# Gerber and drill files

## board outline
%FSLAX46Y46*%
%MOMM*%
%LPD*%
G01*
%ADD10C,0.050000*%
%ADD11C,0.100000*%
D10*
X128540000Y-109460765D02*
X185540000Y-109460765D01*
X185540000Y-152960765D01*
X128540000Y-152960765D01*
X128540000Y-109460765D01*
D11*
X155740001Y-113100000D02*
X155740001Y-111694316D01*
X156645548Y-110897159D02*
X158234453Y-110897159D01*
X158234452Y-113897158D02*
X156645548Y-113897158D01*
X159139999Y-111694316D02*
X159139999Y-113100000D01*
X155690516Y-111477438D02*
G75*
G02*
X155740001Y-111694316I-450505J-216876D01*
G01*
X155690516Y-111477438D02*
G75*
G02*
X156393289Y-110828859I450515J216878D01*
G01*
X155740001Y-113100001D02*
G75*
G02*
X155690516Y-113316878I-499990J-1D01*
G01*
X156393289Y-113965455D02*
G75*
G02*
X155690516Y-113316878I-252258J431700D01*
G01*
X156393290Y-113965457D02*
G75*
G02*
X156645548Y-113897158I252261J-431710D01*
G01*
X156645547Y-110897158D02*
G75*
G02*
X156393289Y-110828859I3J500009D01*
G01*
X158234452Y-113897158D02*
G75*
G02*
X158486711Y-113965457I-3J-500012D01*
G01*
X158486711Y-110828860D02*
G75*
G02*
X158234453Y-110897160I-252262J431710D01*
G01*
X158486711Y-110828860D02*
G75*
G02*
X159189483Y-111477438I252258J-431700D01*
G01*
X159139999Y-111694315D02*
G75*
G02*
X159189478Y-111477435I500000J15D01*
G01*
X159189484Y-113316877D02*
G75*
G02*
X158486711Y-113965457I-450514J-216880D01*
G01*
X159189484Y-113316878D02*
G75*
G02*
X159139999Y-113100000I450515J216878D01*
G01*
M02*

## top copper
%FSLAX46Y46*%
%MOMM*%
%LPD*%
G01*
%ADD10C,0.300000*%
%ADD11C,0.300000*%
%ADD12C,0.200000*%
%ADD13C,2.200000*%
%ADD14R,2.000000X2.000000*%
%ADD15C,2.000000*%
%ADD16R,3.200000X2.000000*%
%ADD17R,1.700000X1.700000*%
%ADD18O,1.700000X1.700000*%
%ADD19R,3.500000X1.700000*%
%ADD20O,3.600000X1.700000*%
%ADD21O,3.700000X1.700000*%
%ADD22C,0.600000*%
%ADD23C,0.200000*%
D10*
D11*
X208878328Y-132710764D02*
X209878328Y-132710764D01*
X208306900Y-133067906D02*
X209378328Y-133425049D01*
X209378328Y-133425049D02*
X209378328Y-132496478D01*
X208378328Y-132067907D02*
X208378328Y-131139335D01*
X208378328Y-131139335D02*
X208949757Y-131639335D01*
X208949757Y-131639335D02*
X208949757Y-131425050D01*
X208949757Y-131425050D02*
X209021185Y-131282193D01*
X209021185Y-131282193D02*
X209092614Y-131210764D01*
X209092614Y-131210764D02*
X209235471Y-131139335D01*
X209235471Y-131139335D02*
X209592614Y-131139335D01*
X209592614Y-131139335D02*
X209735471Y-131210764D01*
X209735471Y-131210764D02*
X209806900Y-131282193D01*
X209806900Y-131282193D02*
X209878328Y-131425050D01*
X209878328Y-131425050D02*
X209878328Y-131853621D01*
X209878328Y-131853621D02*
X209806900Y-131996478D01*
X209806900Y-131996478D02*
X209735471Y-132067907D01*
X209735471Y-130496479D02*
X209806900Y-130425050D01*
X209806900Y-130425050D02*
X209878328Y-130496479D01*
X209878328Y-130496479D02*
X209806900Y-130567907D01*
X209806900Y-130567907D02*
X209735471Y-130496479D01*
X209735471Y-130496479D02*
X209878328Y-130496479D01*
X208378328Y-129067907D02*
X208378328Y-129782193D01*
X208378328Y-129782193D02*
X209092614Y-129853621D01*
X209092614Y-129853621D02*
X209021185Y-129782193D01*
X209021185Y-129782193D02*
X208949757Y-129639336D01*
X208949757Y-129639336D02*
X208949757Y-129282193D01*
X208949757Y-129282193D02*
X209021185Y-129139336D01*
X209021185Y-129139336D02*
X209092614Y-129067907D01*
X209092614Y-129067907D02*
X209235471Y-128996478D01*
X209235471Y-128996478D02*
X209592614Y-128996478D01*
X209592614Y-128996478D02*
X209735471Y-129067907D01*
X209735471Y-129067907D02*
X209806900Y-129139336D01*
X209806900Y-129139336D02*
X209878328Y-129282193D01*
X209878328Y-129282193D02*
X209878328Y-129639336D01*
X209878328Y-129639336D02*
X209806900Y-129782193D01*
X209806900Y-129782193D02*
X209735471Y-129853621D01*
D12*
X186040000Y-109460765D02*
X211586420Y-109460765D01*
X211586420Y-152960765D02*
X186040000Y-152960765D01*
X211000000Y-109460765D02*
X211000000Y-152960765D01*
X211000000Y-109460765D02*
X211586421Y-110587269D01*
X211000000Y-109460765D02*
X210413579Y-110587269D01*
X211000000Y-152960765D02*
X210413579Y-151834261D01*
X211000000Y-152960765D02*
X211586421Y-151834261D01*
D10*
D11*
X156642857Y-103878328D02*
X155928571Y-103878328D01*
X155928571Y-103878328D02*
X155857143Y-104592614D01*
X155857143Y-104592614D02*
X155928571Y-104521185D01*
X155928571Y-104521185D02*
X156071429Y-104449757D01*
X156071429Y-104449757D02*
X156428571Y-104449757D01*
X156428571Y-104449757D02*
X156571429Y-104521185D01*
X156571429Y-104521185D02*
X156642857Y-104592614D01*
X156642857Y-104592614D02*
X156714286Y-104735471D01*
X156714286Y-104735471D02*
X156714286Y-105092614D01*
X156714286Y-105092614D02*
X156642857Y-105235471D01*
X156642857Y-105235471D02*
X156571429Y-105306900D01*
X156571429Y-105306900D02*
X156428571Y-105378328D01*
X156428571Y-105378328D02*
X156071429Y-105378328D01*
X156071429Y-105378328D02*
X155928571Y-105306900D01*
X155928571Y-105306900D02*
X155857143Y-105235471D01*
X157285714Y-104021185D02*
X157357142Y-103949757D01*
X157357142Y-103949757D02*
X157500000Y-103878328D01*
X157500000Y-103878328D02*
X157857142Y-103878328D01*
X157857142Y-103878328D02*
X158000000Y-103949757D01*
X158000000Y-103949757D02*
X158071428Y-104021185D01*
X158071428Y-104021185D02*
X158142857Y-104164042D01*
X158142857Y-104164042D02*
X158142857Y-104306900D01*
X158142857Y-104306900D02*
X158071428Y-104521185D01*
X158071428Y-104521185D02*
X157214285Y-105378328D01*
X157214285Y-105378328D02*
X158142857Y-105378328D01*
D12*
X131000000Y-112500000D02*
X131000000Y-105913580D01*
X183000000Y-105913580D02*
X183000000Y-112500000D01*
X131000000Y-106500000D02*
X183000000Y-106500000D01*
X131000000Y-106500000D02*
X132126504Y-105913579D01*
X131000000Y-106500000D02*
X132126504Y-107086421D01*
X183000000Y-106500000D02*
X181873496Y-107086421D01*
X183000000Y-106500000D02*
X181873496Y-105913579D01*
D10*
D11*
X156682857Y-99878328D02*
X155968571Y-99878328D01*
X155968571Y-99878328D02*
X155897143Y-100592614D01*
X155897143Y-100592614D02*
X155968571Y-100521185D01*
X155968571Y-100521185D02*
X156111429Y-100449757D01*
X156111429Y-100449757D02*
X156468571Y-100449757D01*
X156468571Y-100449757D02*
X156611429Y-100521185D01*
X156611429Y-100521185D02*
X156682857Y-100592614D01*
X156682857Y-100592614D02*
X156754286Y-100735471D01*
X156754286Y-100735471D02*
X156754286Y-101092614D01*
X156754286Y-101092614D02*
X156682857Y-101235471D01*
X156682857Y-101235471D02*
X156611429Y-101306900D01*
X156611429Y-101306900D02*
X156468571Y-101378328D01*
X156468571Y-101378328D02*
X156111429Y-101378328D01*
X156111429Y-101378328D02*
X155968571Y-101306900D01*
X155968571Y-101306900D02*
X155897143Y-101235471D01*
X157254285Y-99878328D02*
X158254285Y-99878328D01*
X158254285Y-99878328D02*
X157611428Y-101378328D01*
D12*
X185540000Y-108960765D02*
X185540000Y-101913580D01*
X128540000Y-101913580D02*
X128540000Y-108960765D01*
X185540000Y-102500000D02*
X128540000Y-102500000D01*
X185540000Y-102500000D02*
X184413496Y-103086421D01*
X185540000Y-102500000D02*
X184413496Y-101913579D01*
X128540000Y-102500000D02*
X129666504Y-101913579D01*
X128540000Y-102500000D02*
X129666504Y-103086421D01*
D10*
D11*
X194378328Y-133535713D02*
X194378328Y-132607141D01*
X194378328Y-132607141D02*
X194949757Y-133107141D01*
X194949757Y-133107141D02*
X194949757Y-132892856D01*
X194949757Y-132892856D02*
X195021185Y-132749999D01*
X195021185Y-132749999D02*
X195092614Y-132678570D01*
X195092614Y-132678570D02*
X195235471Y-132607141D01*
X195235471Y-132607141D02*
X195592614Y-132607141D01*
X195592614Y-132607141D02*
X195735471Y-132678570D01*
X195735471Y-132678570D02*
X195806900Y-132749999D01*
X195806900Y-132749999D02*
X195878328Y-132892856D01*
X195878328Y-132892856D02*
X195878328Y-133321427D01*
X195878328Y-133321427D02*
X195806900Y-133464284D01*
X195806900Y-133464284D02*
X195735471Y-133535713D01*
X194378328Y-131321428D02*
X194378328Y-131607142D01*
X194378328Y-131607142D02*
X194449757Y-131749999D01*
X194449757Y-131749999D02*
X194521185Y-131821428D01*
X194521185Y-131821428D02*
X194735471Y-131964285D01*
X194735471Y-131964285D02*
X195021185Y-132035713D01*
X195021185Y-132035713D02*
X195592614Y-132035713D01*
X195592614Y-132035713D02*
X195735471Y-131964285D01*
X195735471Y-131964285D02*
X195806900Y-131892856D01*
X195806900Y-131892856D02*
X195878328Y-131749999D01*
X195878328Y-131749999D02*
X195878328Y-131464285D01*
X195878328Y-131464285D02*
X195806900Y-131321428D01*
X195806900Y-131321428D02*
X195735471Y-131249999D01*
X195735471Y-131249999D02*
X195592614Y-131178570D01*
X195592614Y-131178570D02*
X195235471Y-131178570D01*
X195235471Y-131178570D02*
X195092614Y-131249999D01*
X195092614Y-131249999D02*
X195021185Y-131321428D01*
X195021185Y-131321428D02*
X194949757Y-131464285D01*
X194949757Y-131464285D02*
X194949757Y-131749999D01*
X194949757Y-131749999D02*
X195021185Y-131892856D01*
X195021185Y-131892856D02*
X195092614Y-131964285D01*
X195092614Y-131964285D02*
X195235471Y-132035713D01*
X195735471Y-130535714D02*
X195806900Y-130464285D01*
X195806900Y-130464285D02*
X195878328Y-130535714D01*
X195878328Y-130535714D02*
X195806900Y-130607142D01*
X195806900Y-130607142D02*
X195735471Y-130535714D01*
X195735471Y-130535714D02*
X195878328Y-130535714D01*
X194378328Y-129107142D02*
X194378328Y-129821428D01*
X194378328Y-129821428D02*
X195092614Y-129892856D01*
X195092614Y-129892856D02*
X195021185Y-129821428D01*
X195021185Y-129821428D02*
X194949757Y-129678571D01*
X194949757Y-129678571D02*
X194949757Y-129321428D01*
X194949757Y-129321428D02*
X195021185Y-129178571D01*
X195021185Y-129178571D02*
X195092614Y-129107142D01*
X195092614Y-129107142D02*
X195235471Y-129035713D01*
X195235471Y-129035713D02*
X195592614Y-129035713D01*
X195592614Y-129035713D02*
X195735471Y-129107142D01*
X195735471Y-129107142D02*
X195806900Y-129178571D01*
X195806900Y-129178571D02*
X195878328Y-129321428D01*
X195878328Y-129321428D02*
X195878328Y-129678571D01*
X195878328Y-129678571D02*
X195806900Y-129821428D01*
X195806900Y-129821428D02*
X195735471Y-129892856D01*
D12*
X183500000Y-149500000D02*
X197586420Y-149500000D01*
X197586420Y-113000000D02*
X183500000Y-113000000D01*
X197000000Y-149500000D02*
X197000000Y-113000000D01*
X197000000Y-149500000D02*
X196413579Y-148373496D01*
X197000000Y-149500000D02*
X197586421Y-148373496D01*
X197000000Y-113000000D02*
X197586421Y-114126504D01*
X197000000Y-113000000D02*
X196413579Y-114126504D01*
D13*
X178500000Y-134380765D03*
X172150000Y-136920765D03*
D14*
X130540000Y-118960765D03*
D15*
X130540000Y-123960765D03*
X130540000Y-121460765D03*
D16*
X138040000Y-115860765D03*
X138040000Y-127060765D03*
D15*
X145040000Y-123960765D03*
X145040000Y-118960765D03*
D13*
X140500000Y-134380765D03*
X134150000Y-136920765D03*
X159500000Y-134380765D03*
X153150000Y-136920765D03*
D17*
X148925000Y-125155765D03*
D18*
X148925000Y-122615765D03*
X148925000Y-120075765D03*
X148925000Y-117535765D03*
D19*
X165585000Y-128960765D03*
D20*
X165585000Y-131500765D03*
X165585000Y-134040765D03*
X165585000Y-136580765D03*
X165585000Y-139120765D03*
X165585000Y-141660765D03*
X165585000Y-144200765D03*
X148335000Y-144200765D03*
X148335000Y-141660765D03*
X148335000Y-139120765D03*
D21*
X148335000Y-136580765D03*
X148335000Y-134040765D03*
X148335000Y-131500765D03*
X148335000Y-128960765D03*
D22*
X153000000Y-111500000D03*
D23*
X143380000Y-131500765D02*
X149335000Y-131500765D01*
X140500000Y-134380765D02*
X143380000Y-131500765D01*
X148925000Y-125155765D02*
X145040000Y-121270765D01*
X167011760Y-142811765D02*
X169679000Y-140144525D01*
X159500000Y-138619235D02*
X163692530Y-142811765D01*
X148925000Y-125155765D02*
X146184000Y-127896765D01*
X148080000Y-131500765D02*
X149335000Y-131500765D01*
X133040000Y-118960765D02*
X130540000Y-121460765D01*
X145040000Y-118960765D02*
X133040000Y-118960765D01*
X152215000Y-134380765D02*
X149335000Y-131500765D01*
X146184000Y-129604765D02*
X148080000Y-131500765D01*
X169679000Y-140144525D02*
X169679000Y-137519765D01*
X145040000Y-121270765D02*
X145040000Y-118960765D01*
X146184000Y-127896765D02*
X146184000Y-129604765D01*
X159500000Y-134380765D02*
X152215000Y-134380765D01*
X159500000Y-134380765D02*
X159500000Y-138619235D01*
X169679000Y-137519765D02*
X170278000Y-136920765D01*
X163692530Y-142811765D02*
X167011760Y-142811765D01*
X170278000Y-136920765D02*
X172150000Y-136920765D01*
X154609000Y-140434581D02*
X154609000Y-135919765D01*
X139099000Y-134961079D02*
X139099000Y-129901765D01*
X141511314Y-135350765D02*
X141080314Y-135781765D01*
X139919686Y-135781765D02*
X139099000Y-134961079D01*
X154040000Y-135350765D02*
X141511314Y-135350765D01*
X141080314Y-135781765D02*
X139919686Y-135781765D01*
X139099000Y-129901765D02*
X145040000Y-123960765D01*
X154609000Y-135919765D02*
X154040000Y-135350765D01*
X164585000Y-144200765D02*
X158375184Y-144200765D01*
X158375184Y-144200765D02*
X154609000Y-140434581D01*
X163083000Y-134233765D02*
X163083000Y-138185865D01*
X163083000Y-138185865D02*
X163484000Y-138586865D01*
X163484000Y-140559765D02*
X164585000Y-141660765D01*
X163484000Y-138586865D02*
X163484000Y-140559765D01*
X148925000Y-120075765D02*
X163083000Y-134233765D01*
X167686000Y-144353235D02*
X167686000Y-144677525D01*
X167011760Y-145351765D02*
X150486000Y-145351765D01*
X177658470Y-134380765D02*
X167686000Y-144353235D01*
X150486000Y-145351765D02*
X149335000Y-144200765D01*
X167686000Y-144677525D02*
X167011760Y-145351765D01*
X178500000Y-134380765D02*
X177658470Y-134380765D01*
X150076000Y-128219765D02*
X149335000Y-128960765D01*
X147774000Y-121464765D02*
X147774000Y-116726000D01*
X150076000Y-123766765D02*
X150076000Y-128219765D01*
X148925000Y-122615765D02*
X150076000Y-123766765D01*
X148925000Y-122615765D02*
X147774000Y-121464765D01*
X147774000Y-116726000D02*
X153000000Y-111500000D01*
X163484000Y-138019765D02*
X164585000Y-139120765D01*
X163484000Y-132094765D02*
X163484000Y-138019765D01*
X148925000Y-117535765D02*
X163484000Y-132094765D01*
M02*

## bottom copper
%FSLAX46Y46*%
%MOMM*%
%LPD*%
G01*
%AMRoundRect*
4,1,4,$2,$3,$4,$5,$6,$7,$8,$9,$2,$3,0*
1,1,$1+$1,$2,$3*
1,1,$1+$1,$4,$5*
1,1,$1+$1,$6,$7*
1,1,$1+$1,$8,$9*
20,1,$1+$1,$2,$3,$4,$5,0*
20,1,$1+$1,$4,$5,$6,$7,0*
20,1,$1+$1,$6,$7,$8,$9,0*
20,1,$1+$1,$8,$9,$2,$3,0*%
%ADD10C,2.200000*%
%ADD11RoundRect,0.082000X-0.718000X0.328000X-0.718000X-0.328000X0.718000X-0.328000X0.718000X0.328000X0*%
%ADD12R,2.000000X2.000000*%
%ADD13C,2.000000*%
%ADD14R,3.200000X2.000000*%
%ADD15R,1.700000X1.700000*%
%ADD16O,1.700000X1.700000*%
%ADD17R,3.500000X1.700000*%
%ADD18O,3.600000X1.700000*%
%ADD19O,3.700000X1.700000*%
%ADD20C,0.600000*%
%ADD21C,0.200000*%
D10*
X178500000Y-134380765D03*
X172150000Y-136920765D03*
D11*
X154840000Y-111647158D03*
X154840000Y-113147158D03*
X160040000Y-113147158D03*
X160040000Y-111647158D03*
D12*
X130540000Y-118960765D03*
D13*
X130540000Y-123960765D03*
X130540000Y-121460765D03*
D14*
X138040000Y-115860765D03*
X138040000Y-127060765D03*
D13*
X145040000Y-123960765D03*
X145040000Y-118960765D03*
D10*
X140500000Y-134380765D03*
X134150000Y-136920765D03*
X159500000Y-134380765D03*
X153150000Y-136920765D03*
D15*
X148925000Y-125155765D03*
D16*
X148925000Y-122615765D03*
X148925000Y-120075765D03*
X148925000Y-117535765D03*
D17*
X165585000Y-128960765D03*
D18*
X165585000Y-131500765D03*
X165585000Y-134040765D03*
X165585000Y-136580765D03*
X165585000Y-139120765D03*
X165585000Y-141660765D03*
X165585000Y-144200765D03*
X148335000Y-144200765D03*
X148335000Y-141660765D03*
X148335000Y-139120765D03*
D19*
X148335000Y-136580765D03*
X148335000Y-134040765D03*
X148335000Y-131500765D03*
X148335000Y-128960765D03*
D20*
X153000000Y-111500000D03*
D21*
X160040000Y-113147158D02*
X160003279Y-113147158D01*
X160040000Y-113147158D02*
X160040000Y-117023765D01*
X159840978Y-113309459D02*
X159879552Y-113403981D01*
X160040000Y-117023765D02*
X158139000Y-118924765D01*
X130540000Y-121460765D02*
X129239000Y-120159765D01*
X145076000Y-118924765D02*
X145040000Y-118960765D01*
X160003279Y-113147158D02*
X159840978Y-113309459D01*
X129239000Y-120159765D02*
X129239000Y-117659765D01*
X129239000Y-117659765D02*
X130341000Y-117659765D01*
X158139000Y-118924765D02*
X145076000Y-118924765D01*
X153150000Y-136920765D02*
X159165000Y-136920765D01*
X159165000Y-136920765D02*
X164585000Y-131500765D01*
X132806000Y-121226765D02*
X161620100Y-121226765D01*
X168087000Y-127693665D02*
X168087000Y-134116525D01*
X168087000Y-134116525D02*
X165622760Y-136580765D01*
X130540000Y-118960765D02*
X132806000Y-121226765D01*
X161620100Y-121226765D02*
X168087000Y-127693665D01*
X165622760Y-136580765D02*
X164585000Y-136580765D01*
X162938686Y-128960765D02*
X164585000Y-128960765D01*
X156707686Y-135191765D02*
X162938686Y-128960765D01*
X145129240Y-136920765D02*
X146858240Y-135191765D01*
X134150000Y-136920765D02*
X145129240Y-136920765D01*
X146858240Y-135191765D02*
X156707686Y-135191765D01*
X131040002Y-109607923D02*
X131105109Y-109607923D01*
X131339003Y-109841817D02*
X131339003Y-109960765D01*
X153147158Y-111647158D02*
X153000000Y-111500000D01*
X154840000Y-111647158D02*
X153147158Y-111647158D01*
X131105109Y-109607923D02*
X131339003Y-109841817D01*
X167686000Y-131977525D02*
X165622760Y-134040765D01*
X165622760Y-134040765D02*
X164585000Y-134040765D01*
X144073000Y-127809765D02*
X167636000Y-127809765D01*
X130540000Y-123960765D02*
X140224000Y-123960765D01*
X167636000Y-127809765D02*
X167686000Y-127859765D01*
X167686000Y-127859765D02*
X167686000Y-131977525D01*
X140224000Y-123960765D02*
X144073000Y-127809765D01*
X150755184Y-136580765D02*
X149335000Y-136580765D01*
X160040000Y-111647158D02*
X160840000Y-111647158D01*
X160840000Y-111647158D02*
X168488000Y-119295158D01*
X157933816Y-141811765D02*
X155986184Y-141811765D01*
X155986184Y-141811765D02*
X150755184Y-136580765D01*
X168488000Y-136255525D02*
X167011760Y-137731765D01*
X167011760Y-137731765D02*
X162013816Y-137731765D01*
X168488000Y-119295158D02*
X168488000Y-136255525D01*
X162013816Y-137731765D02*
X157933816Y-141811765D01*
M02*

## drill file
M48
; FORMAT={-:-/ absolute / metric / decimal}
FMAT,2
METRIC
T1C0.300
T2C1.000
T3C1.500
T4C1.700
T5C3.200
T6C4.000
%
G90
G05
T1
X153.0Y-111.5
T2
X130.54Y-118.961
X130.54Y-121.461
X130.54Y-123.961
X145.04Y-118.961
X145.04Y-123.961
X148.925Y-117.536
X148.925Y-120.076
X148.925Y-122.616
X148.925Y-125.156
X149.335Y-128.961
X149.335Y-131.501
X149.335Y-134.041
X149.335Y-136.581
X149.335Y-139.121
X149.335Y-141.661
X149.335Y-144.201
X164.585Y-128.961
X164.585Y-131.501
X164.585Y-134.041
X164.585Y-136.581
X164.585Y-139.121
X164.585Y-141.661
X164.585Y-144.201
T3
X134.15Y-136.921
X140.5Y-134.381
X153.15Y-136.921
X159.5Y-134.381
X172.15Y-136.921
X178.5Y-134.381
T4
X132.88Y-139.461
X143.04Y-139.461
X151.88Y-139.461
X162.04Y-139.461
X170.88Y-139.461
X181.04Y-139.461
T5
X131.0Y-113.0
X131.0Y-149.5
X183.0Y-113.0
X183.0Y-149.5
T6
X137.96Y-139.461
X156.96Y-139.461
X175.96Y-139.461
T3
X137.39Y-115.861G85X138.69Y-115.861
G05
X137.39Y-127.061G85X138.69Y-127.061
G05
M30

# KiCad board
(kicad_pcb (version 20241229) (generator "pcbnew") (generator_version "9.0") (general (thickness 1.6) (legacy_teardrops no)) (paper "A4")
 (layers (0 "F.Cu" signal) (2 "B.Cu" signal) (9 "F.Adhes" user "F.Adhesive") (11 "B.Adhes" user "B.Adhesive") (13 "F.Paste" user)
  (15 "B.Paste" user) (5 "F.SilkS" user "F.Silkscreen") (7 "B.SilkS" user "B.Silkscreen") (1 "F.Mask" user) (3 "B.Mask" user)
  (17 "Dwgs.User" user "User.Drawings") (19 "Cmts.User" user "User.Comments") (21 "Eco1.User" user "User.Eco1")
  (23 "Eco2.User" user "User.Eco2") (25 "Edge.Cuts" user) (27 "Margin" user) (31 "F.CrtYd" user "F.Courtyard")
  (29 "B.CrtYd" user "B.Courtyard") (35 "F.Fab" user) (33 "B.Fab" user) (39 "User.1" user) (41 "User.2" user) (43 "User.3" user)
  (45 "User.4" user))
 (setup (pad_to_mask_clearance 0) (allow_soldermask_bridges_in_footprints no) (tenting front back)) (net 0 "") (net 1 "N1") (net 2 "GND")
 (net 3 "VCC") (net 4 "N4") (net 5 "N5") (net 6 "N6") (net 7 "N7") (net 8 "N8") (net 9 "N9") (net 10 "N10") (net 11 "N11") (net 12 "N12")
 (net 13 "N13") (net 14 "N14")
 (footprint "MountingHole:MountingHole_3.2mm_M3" (layer "F.Cu") (at 183 149.5)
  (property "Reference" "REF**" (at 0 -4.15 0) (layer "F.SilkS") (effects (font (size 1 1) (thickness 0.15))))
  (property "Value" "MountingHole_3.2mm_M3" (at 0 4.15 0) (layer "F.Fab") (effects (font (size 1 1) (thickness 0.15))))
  (pad "" np_thru_hole circle (at 0 0) (size 3.2 3.2) (drill 3.2) (layers "*.Cu" "*.Mask")))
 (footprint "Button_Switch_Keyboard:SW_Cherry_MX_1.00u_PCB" (layer "F.Cu") (at 178.5 134.380765)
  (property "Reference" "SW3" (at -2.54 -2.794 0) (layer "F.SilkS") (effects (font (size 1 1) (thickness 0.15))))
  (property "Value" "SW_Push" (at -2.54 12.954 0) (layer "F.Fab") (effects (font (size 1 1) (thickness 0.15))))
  (pad "" np_thru_hole circle (at -7.62 5.08) (size 1.7 1.7) (drill 1.7) (layers "*.Cu" "*.Mask"))
  (pad "" np_thru_hole circle (at -2.54 5.08) (size 4 4) (drill 4) (layers "*.Cu" "*.Mask"))
  (pad "" np_thru_hole circle (at 2.54 5.08) (size 1.7 1.7) (drill 1.7) (layers "*.Cu" "*.Mask"))
  (pad "1" thru_hole circle (at 0 0) (size 2.2 2.2) (drill 1.5) (layers "*.Cu" "*.Mask") (remove_unused_layers no) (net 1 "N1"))
  (pad "2" thru_hole circle (at -6.35 2.54) (size 2.2 2.2) (drill 1.5) (layers "*.Cu" "*.Mask") (remove_unused_layers no) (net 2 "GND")))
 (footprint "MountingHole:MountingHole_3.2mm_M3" (layer "F.Cu") (at 131 149.5)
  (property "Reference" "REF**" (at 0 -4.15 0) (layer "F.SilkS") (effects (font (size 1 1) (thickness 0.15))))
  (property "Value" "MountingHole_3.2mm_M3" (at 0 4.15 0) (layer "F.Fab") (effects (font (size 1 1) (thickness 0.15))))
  (pad "" np_thru_hole circle (at 0 0) (size 3.2 3.2) (drill 3.2) (layers "*.Cu" "*.Mask")))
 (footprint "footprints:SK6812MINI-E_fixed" (layer "F.Cu") (at 157.439999 112.5)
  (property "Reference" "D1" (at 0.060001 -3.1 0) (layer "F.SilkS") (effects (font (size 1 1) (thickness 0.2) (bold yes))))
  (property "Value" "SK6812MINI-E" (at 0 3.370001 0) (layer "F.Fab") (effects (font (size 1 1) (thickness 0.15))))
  (fp_line (start -1.699998 0.6) (end -1.699998 -0.805684) (stroke (width 0.1) (type solid)) (layer "Edge.Cuts"))
  (fp_line (start -0.794451 -1.602841) (end 0.794454 -1.602841) (stroke (width 0.1) (type solid)) (layer "Edge.Cuts"))
  (fp_line (start 0.794453 1.397158) (end -0.794451 1.397158) (stroke (width 0.1) (type solid)) (layer "Edge.Cuts"))
  (fp_line (start 1.7 -0.805684) (end 1.7 0.6) (stroke (width 0.1) (type solid)) (layer "Edge.Cuts"))
  (fp_arc (start -1.749483 -1.022562) (mid -1.712526 -0.91691) (end -1.699998 -0.805684) (stroke (width 0.1) (type solid))
   (layer "Edge.Cuts"))
  (fp_arc (start -1.749483 -1.022562) (mid -1.63807 -1.606877) (end -1.04671 -1.671141) (stroke (width 0.1) (type solid))
   (layer "Edge.Cuts"))
  (fp_arc (start -1.699998 0.600001) (mid -1.712526 0.711226) (end -1.749483 0.816878) (stroke (width 0.1) (type solid)) (layer "Edge.Cuts"))
  (fp_arc (start -1.04671 1.465455) (mid -1.638069 1.401192) (end -1.749483 0.816878) (stroke (width 0.1) (type solid)) (layer "Edge.Cuts"))
  (fp_arc (start -1.046709 1.465457) (mid -0.925121 1.414535) (end -0.794451 1.397158) (stroke (width 0.1) (type solid)) (layer "Edge.Cuts"))
  (fp_arc (start -0.794452 -1.602842) (mid -0.925122 -1.620219) (end -1.04671 -1.671141) (stroke (width 0.1) (type solid))
   (layer "Edge.Cuts"))
  (fp_arc (start 0.794453 1.397158) (mid 0.925124 1.414535) (end 1.046712 1.465457) (stroke (width 0.1) (type solid)) (layer "Edge.Cuts"))
  (fp_arc (start 1.046712 -1.67114) (mid 0.925124 -1.620218) (end 0.794454 -1.602841) (stroke (width 0.1) (type solid)) (layer "Edge.Cuts"))
  (fp_arc (start 1.046712 -1.67114) (mid 1.638072 -1.606876) (end 1.749485 -1.022562) (stroke (width 0.1) (type solid)) (layer "Edge.Cuts"))
  (fp_arc (start 1.7 -0.805685) (mid 1.712528 -0.91691) (end 1.749485 -1.022562) (stroke (width 0.1) (type solid)) (layer "Edge.Cuts"))
  (fp_arc (start 1.749485 0.816877) (mid 1.638073 1.401193) (end 1.046712 1.465457) (stroke (width 0.1) (type solid)) (layer "Edge.Cuts"))
  (fp_arc (start 1.749485 0.816878) (mid 1.712528 0.711226) (end 1.7 0.6) (stroke (width 0.1) (type solid)) (layer "Edge.Cuts"))
  (pad "1" smd roundrect (at -2.599999 -0.852842 270) (size 0.82 1.6) (layers "B.Cu" "B.Mask" "B.Paste") (roundrect_rratio 0.1)
   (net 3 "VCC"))
  (pad "2" smd roundrect (at -2.599999 0.647158 270) (size 0.82 1.6) (layers "B.Cu" "B.Mask" "B.Paste") (roundrect_rratio 0.1))
  (pad "3" smd roundrect (at 2.600001 0.647158 270) (size 0.82 1.6) (layers "B.Cu" "B.Mask" "B.Paste") (roundrect_rratio 0.1) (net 2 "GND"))
  (pad "4" smd roundrect (at 2.600001 -0.852842 270) (size 0.82 1.6) (layers "B.Cu" "B.Mask" "B.Paste") (roundrect_rratio 0.1) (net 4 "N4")))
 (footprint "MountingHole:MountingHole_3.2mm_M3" (layer "F.Cu") (at 131 113)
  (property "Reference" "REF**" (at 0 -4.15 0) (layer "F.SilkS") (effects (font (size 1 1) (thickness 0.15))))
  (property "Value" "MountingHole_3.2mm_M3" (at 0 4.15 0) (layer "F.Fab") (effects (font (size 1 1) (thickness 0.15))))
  (pad "" np_thru_hole circle (at 0 0) (size 3.2 3.2) (drill 3.2) (layers "*.Cu" "*.Mask")))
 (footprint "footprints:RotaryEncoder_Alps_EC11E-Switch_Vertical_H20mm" (layer "F.Cu") (at 130.54 118.960765)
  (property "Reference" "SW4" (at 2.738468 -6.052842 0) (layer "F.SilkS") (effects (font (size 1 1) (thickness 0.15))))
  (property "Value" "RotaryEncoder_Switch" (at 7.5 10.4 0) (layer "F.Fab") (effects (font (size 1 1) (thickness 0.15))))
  (pad "A" thru_hole rect (at 0 0) (size 2 2) (drill 1) (layers "*.Cu" "*.Mask") (remove_unused_layers no) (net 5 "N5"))
  (pad "B" thru_hole circle (at 0 5) (size 2 2) (drill 1) (layers "*.Cu" "*.Mask") (remove_unused_layers no) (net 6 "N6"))
  (pad "C" thru_hole circle (at 0 2.5) (size 2 2) (drill 1) (layers "*.Cu" "*.Mask") (remove_unused_layers no) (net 2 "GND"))
  (pad "MP" thru_hole rect (at 7.5 -3.1) (size 3.2 2) (drill oval 2.8 1.5) (layers "*.Cu" "*.Mask") (remove_unused_layers no))
  (pad "MP" thru_hole rect (at 7.5 8.1) (size 3.2 2) (drill oval 2.8 1.5) (layers "*.Cu" "*.Mask") (remove_unused_layers no))
  (pad "S1" thru_hole circle (at 14.5 5) (size 2 2) (drill 1) (layers "*.Cu" "*.Mask") (remove_unused_layers no) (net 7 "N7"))
  (pad "S2" thru_hole circle (at 14.5 0) (size 2 2) (drill 1) (layers "*.Cu" "*.Mask") (remove_unused_layers no) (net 2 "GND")))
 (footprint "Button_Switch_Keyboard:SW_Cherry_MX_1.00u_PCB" (layer "F.Cu") (at 140.5 134.380765)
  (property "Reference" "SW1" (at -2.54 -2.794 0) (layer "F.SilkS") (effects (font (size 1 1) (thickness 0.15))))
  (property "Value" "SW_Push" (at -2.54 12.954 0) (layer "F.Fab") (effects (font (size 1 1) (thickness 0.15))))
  (pad "" np_thru_hole circle (at -7.62 5.08) (size 1.7 1.7) (drill 1.7) (layers "*.Cu" "*.Mask"))
  (pad "" np_thru_hole circle (at -2.54 5.08) (size 4 4) (drill 4) (layers "*.Cu" "*.Mask"))
  (pad "" np_thru_hole circle (at 2.54 5.08) (size 1.7 1.7) (drill 1.7) (layers "*.Cu" "*.Mask"))
  (pad "1" thru_hole circle (at 0 0) (size 2.2 2.2) (drill 1.5) (layers "*.Cu" "*.Mask") (remove_unused_layers no) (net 2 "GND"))
  (pad "2" thru_hole circle (at -6.35 2.54) (size 2.2 2.2) (drill 1.5) (layers "*.Cu" "*.Mask") (remove_unused_layers no) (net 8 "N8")))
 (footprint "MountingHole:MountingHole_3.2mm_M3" (layer "F.Cu") (at 183 113)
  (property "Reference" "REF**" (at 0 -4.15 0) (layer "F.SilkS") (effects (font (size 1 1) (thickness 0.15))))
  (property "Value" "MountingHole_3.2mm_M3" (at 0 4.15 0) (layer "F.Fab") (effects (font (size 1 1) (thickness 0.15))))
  (pad "" np_thru_hole circle (at 0 0) (size 3.2 3.2) (drill 3.2) (layers "*.Cu" "*.Mask")))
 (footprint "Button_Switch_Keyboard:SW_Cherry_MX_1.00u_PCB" (layer "F.Cu") (at 159.5 134.380765)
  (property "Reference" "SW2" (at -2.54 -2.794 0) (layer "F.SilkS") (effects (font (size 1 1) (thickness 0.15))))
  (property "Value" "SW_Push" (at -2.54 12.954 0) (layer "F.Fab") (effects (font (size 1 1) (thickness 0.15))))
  (pad "" np_thru_hole circle (at -7.62 5.08) (size 1.7 1.7) (drill 1.7) (layers "*.Cu" "*.Mask"))
  (pad "" np_thru_hole circle (at -2.54 5.08) (size 4 4) (drill 4) (layers "*.Cu" "*.Mask"))
  (pad "" np_thru_hole circle (at 2.54 5.08) (size 1.7 1.7) (drill 1.7) (layers "*.Cu" "*.Mask"))
  (pad "1" thru_hole circle (at 0 0) (size 2.2 2.2) (drill 1.5) (layers "*.Cu" "*.Mask") (remove_unused_layers no) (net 2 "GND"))
  (pad "2" thru_hole circle (at -6.35 2.54) (size 2.2 2.2) (drill 1.5) (layers "*.Cu" "*.Mask") (remove_unused_layers no) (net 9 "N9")))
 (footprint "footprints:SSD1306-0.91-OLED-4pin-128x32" (layer "F.Cu") (at 185.425 127.345765 180)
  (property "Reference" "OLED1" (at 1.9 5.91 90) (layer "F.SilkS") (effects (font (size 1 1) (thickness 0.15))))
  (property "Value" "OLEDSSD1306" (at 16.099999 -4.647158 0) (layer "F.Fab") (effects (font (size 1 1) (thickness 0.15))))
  (pad "1" thru_hole rect (at 36.5 2.19 180) (size 1.7 1.7) (drill 1) (layers "*.Cu" "*.Mask") (remove_unused_layers no) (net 2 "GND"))
  (pad "2" thru_hole oval (at 36.5 4.73 180) (size 1.7 1.7) (drill 1) (layers "*.Cu" "*.Mask") (remove_unused_layers no) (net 3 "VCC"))
  (pad "3" thru_hole oval (at 36.5 7.27 180) (size 1.7 1.7) (drill 1) (layers "*.Cu" "*.Mask") (remove_unused_layers no) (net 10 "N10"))
  (pad "4" thru_hole oval (at 36.5 9.81 180) (size 1.7 1.7) (drill 1) (layers "*.Cu" "*.Mask") (remove_unused_layers no) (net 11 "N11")))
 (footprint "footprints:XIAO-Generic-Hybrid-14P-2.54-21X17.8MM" (layer "B.Cu") (at 156.96 136.580765 180)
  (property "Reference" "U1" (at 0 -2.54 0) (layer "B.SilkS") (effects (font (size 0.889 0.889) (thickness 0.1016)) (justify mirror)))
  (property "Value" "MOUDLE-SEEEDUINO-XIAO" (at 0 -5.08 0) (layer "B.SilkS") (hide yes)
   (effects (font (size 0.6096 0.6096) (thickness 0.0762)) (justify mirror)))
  (pad "1" thru_hole rect (at -7.625 7.62 180) (size 3.5 1.7) (drill 1 (offset -1 0)) (layers "*.Cu" "*.Mask") (remove_unused_layers no)
   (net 8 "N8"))
  (pad "2" thru_hole oval (at -7.625 5.08 180) (size 3.6 1.7) (drill 1 (offset -1 0)) (layers "*.Cu" "*.Mask") (remove_unused_layers no)
   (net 9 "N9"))
  (pad "3" thru_hole oval (at -7.625 2.54 180) (size 3.6 1.7) (drill 1 (offset -1 0)) (layers "*.Cu" "*.Mask") (remove_unused_layers no)
   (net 6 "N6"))
  (pad "4" thru_hole oval (at -7.625 0 180) (size 3.6 1.7) (drill 1 (offset -1 0)) (layers "*.Cu" "*.Mask") (remove_unused_layers no)
   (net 5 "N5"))
  (pad "5" thru_hole oval (at -7.625 -2.54 180) (size 3.6 1.7) (drill 1 (offset -1 0)) (layers "*.Cu" "*.Mask") (remove_unused_layers no)
   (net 11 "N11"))
  (pad "6" thru_hole oval (at -7.625 -5.08) (size 3.6 1.7) (drill 1 (offset 1 0)) (layers "*.Cu" "*.Mask") (remove_unused_layers no)
   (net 10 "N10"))
  (pad "7" thru_hole oval (at -7.625 -7.62 180) (size 3.6 1.7) (drill 1 (offset -1 0)) (layers "*.Cu" "*.Mask") (remove_unused_layers no)
   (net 7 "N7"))
  (pad "8" thru_hole oval (at 7.625 -7.62 180) (size 3.6 1.7) (drill 1 (offset 1 0)) (layers "*.Cu" "*.Mask") (remove_unused_layers no)
   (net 1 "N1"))
  (pad "9" thru_hole oval (at 7.625 -5.08 180) (size 3.6 1.7) (drill 1 (offset 1 0)) (layers "*.Cu" "*.Mask") (remove_unused_layers no)
   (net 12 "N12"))
  (pad "10" thru_hole oval (at 7.625 -2.54 180) (size 3.6 1.7) (drill 1 (offset 1 0)) (layers "*.Cu" "*.Mask") (remove_unused_layers no)
   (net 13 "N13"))
  (pad "11" thru_hole oval (at 7.625 0 180) (size 3.7 1.7) (drill 1 (offset 1 0)) (layers "*.Cu" "*.Mask") (remove_unused_layers no)
   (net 4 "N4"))
  (pad "12" thru_hole oval (at 7.625 2.54 180) (size 3.7 1.7) (drill 1 (offset 1 0)) (layers "*.Cu" "*.Mask") (remove_unused_layers no)
   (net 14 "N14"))
  (pad "13" thru_hole oval (at 7.625 5.08 180) (size 3.7 1.7) (drill 1 (offset 1 0)) (layers "*.Cu" "*.Mask") (remove_unused_layers no)
   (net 2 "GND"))
  (pad "14" thru_hole oval (at 7.625 7.62 180) (size 3.7 1.7) (drill 1 (offset 1 0)) (layers "*.Cu" "*.Mask") (remove_unused_layers no)
   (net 3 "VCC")))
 (gr_rect (start 128.54 109.460765) (end 185.54 152.960765) (stroke (width 0.05) (type default)) (fill no) (layer "Edge.Cuts"))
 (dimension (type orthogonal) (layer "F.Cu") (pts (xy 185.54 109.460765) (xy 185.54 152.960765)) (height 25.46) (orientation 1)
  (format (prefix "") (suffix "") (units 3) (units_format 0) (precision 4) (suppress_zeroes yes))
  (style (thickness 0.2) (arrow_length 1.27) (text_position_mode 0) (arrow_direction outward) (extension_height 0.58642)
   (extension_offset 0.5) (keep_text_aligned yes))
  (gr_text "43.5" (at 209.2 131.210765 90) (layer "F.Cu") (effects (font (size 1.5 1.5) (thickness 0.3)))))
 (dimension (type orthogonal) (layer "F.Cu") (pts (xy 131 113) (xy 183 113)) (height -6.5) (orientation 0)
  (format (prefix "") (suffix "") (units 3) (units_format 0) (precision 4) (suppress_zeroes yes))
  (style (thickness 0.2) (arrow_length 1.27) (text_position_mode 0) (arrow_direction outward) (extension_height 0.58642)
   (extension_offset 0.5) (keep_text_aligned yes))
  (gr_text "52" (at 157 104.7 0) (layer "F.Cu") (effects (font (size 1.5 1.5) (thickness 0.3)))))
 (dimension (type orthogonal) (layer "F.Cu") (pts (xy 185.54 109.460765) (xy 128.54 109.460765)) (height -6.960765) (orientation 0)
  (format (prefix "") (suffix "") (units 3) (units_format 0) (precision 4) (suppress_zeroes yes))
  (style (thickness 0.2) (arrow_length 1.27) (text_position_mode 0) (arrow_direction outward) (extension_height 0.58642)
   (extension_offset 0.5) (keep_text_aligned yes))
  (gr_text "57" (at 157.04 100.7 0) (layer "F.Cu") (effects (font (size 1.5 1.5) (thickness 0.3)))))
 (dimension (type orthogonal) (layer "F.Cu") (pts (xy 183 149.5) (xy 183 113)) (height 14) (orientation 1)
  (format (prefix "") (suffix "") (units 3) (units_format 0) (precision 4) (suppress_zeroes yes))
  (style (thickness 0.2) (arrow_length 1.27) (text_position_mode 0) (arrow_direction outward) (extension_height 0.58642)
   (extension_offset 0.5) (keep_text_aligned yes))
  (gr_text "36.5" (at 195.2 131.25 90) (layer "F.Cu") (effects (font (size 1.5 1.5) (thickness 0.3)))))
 (segment (start 143.38 131.500765) (end 149.335 131.500765) (width 0.2) (layer "F.Cu") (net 2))
 (segment (start 140.5 134.380765) (end 143.38 131.500765) (width 0.2) (layer "F.Cu") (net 2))
 (segment (start 148.925 125.155765) (end 145.04 121.270765) (width 0.2) (layer "F.Cu") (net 2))
 (segment (start 167.01176 142.811765) (end 169.679 140.144525) (width 0.2) (layer "F.Cu") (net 2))
 (segment (start 159.5 138.619235) (end 163.69253 142.811765) (width 0.2) (layer "F.Cu") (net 2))
 (segment (start 148.925 125.155765) (end 146.184 127.896765) (width 0.2) (layer "F.Cu") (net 2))
 (segment (start 148.08 131.500765) (end 149.335 131.500765) (width 0.2) (layer "F.Cu") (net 2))
 (segment (start 133.04 118.960765) (end 130.54 121.460765) (width 0.2) (layer "F.Cu") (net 2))
 (segment (start 145.04 118.960765) (end 133.04 118.960765) (width 0.2) (layer "F.Cu") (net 2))
 (segment (start 152.215 134.380765) (end 149.335 131.500765) (width 0.2) (layer "F.Cu") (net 2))
 (segment (start 146.184 129.604765) (end 148.08 131.500765) (width 0.2) (layer "F.Cu") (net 2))
 (segment (start 169.679 140.144525) (end 169.679 137.519765) (width 0.2) (layer "F.Cu") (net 2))
 (segment (start 145.04 121.270765) (end 145.04 118.960765) (width 0.2) (layer "F.Cu") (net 2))
 (segment (start 146.184 127.896765) (end 146.184 129.604765) (width 0.2) (layer "F.Cu") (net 2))
 (segment (start 159.5 134.380765) (end 152.215 134.380765) (width 0.2) (layer "F.Cu") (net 2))
 (segment (start 159.5 134.380765) (end 159.5 138.619235) (width 0.2) (layer "F.Cu") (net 2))
 (segment (start 169.679 137.519765) (end 170.278 136.920765) (width 0.2) (layer "F.Cu") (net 2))
 (segment (start 163.69253 142.811765) (end 167.01176 142.811765) (width 0.2) (layer "F.Cu") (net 2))
 (segment (start 170.278 136.920765) (end 172.15 136.920765) (width 0.2) (layer "F.Cu") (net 2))
 (segment (start 160.04 113.147158) (end 160.003279 113.147158) (width 0.2) (layer "B.Cu") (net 2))
 (segment (start 160.04 113.147158) (end 160.04 117.023765) (width 0.2) (layer "B.Cu") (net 2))
 (segment (start 159.840978 113.309459) (end 159.879552 113.403981) (width 0.2) (layer "B.Cu") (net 2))
 (segment (start 160.04 117.023765) (end 158.139 118.924765) (width 0.2) (layer "B.Cu") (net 2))
 (segment (start 130.54 121.460765) (end 129.239 120.159765) (width 0.2) (layer "B.Cu") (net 2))
 (segment (start 145.076 118.924765) (end 145.04 118.960765) (width 0.2) (layer "B.Cu") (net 2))
 (segment (start 160.003279 113.147158) (end 159.840978 113.309459) (width 0.2) (layer "B.Cu") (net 2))
 (segment (start 129.239 120.159765) (end 129.239 117.659765) (width 0.2) (layer "B.Cu") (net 2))
 (segment (start 129.239 117.659765) (end 130.341 117.659765) (width 0.2) (layer "B.Cu") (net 2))
 (segment (start 158.139 118.924765) (end 145.076 118.924765) (width 0.2) (layer "B.Cu") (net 2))
 (segment (start 154.609 140.434581) (end 154.609 135.919765) (width 0.2) (layer "F.Cu") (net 7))
 (segment (start 139.099 134.961079) (end 139.099 129.901765) (width 0.2) (layer "F.Cu") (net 7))
 (segment (start 141.511314 135.350765) (end 141.080314 135.781765) (width 0.2) (layer "F.Cu") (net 7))
 (segment (start 139.919686 135.781765) (end 139.099 134.961079) (width 0.2) (layer "F.Cu") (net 7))
 (segment (start 154.04 135.350765) (end 141.511314 135.350765) (width 0.2) (layer "F.Cu") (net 7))
 (segment (start 141.080314 135.781765) (end 139.919686 135.781765) (width 0.2) (layer "F.Cu") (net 7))
 (segment (start 139.099 129.901765) (end 145.04 123.960765) (width 0.2) (layer "F.Cu") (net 7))
 (segment (start 154.609 135.919765) (end 154.04 135.350765) (width 0.2) (layer "F.Cu") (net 7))
 (segment (start 164.585 144.200765) (end 158.375184 144.200765) (width 0.2) (layer "F.Cu") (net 7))
 (segment (start 158.375184 144.200765) (end 154.609 140.434581) (width 0.2) (layer "F.Cu") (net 7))
 (segment (start 153.15 136.920765) (end 159.165 136.920765) (width 0.2) (layer "B.Cu") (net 9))
 (segment (start 159.165 136.920765) (end 164.585 131.500765) (width 0.2) (layer "B.Cu") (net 9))
 (segment (start 132.806 121.226765) (end 161.6201 121.226765) (width 0.2) (layer "B.Cu") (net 5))
 (segment (start 168.087 127.693665) (end 168.087 134.116525) (width 0.2) (layer "B.Cu") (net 5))
 (segment (start 168.087 134.116525) (end 165.62276 136.580765) (width 0.2) (layer "B.Cu") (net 5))
 (segment (start 130.54 118.960765) (end 132.806 121.226765) (width 0.2) (layer "B.Cu") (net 5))
 (segment (start 161.6201 121.226765) (end 168.087 127.693665) (width 0.2) (layer "B.Cu") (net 5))
 (segment (start 165.62276 136.580765) (end 164.585 136.580765) (width 0.2) (layer "B.Cu") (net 5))
 (segment (start 163.083 134.233765) (end 163.083 138.185865) (width 0.2) (layer "F.Cu") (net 10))
 (segment (start 163.083 138.185865) (end 163.484 138.586865) (width 0.2) (layer "F.Cu") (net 10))
 (segment (start 163.484 140.559765) (end 164.585 141.660765) (width 0.2) (layer "F.Cu") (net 10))
 (segment (start 163.484 138.586865) (end 163.484 140.559765) (width 0.2) (layer "F.Cu") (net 10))
 (segment (start 148.925 120.075765) (end 163.083 134.233765) (width 0.2) (layer "F.Cu") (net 10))
 (segment (start 162.938686 128.960765) (end 164.585 128.960765) (width 0.2) (layer "B.Cu") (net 8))
 (segment (start 156.707686 135.191765) (end 162.938686 128.960765) (width 0.2) (layer "B.Cu") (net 8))
 (segment (start 145.12924 136.920765) (end 146.85824 135.191765) (width 0.2) (layer "B.Cu") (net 8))
 (segment (start 134.15 136.920765) (end 145.12924 136.920765) (width 0.2) (layer "B.Cu") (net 8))
 (segment (start 146.85824 135.191765) (end 156.707686 135.191765) (width 0.2) (layer "B.Cu") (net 8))
 (segment (start 167.686 144.353235) (end 167.686 144.677525) (width 0.2) (layer "F.Cu") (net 1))
 (segment (start 167.01176 145.351765) (end 150.486 145.351765) (width 0.2) (layer "F.Cu") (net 1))
 (segment (start 177.65847 134.380765) (end 167.686 144.353235) (width 0.2) (layer "F.Cu") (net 1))
 (segment (start 150.486 145.351765) (end 149.335 144.200765) (width 0.2) (layer "F.Cu") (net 1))
 (segment (start 167.686 144.677525) (end 167.01176 145.351765) (width 0.2) (layer "F.Cu") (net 1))
 (segment (start 178.5 134.380765) (end 177.65847 134.380765) (width 0.2) (layer "F.Cu") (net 1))
 (segment (start 150.076 128.219765) (end 149.335 128.960765) (width 0.2) (layer "F.Cu") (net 3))
 (segment (start 147.774 121.464765) (end 147.774 116.726) (width 0.2) (layer "F.Cu") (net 3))
 (segment (start 150.076 123.766765) (end 150.076 128.219765) (width 0.2) (layer "F.Cu") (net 3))
 (segment (start 148.925 122.615765) (end 150.076 123.766765) (width 0.2) (layer "F.Cu") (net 3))
 (segment (start 148.925 122.615765) (end 147.774 121.464765) (width 0.2) (layer "F.Cu") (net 3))
 (segment (start 147.774 116.726) (end 153 111.5) (width 0.2) (layer "F.Cu") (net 3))
 (via (at 153 111.5) (size 0.6) (drill 0.3) (layers "F.Cu" "B.Cu") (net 3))
 (segment (start 131.040002 109.607923) (end 131.105109 109.607923) (width 0.2) (layer "B.Cu") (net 3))
 (segment (start 131.339003 109.841817) (end 131.339003 109.960765) (width 0.2) (layer "B.Cu") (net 3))
 (segment (start 153.147158 111.647158) (end 153 111.5) (width 0.2) (layer "B.Cu") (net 3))
 (segment (start 154.84 111.647158) (end 153.147158 111.647158) (width 0.2) (layer "B.Cu") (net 3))
 (segment (start 131.105109 109.607923) (end 131.339003 109.841817) (width 0.2) (layer "B.Cu") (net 3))
 (segment (start 167.686 131.977525) (end 165.62276 134.040765) (width 0.2) (layer "B.Cu") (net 6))
 (segment (start 165.62276 134.040765) (end 164.585 134.040765) (width 0.2) (layer "B.Cu") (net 6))
 (segment (start 144.073 127.809765) (end 167.636 127.809765) (width 0.2) (layer "B.Cu") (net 6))
 (segment (start 130.54 123.960765) (end 140.224 123.960765) (width 0.2) (layer "B.Cu") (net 6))
 (segment (start 167.636 127.809765) (end 167.686 127.859765) (width 0.2) (layer "B.Cu") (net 6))
 (segment (start 167.686 127.859765) (end 167.686 131.977525) (width 0.2) (layer "B.Cu") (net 6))
 (segment (start 140.224 123.960765) (end 144.073 127.809765) (width 0.2) (layer "B.Cu") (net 6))
 (segment (start 163.484 138.019765) (end 164.585 139.120765) (width 0.2) (layer "F.Cu") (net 11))
 (segment (start 163.484 132.094765) (end 163.484 138.019765) (width 0.2) (layer "F.Cu") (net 11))
 (segment (start 148.925 117.535765) (end 163.484 132.094765) (width 0.2) (layer "F.Cu") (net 11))
 (segment (start 150.755184 136.580765) (end 149.335 136.580765) (width 0.2) (layer "B.Cu") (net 4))
 (segment (start 160.04 111.647158) (end 160.84 111.647158) (width 0.2) (layer "B.Cu") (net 4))
 (segment (start 160.84 111.647158) (end 168.488 119.295158) (width 0.2) (layer "B.Cu") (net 4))
 (segment (start 157.933816 141.811765) (end 155.986184 141.811765) (width 0.2) (layer "B.Cu") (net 4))
 (segment (start 155.986184 141.811765) (end 150.755184 136.580765) (width 0.2) (layer "B.Cu") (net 4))
 (segment (start 168.488 136.255525) (end 167.01176 137.731765) (width 0.2) (layer "B.Cu") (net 4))
 (segment (start 167.01176 137.731765) (end 162.013816 137.731765) (width 0.2) (layer "B.Cu") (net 4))
 (segment (start 168.488 119.295158) (end 168.488 136.255525) (width 0.2) (layer "B.Cu") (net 4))
 (segment (start 162.013816 137.731765) (end 157.933816 141.811765) (width 0.2) (layer "B.Cu") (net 4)))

